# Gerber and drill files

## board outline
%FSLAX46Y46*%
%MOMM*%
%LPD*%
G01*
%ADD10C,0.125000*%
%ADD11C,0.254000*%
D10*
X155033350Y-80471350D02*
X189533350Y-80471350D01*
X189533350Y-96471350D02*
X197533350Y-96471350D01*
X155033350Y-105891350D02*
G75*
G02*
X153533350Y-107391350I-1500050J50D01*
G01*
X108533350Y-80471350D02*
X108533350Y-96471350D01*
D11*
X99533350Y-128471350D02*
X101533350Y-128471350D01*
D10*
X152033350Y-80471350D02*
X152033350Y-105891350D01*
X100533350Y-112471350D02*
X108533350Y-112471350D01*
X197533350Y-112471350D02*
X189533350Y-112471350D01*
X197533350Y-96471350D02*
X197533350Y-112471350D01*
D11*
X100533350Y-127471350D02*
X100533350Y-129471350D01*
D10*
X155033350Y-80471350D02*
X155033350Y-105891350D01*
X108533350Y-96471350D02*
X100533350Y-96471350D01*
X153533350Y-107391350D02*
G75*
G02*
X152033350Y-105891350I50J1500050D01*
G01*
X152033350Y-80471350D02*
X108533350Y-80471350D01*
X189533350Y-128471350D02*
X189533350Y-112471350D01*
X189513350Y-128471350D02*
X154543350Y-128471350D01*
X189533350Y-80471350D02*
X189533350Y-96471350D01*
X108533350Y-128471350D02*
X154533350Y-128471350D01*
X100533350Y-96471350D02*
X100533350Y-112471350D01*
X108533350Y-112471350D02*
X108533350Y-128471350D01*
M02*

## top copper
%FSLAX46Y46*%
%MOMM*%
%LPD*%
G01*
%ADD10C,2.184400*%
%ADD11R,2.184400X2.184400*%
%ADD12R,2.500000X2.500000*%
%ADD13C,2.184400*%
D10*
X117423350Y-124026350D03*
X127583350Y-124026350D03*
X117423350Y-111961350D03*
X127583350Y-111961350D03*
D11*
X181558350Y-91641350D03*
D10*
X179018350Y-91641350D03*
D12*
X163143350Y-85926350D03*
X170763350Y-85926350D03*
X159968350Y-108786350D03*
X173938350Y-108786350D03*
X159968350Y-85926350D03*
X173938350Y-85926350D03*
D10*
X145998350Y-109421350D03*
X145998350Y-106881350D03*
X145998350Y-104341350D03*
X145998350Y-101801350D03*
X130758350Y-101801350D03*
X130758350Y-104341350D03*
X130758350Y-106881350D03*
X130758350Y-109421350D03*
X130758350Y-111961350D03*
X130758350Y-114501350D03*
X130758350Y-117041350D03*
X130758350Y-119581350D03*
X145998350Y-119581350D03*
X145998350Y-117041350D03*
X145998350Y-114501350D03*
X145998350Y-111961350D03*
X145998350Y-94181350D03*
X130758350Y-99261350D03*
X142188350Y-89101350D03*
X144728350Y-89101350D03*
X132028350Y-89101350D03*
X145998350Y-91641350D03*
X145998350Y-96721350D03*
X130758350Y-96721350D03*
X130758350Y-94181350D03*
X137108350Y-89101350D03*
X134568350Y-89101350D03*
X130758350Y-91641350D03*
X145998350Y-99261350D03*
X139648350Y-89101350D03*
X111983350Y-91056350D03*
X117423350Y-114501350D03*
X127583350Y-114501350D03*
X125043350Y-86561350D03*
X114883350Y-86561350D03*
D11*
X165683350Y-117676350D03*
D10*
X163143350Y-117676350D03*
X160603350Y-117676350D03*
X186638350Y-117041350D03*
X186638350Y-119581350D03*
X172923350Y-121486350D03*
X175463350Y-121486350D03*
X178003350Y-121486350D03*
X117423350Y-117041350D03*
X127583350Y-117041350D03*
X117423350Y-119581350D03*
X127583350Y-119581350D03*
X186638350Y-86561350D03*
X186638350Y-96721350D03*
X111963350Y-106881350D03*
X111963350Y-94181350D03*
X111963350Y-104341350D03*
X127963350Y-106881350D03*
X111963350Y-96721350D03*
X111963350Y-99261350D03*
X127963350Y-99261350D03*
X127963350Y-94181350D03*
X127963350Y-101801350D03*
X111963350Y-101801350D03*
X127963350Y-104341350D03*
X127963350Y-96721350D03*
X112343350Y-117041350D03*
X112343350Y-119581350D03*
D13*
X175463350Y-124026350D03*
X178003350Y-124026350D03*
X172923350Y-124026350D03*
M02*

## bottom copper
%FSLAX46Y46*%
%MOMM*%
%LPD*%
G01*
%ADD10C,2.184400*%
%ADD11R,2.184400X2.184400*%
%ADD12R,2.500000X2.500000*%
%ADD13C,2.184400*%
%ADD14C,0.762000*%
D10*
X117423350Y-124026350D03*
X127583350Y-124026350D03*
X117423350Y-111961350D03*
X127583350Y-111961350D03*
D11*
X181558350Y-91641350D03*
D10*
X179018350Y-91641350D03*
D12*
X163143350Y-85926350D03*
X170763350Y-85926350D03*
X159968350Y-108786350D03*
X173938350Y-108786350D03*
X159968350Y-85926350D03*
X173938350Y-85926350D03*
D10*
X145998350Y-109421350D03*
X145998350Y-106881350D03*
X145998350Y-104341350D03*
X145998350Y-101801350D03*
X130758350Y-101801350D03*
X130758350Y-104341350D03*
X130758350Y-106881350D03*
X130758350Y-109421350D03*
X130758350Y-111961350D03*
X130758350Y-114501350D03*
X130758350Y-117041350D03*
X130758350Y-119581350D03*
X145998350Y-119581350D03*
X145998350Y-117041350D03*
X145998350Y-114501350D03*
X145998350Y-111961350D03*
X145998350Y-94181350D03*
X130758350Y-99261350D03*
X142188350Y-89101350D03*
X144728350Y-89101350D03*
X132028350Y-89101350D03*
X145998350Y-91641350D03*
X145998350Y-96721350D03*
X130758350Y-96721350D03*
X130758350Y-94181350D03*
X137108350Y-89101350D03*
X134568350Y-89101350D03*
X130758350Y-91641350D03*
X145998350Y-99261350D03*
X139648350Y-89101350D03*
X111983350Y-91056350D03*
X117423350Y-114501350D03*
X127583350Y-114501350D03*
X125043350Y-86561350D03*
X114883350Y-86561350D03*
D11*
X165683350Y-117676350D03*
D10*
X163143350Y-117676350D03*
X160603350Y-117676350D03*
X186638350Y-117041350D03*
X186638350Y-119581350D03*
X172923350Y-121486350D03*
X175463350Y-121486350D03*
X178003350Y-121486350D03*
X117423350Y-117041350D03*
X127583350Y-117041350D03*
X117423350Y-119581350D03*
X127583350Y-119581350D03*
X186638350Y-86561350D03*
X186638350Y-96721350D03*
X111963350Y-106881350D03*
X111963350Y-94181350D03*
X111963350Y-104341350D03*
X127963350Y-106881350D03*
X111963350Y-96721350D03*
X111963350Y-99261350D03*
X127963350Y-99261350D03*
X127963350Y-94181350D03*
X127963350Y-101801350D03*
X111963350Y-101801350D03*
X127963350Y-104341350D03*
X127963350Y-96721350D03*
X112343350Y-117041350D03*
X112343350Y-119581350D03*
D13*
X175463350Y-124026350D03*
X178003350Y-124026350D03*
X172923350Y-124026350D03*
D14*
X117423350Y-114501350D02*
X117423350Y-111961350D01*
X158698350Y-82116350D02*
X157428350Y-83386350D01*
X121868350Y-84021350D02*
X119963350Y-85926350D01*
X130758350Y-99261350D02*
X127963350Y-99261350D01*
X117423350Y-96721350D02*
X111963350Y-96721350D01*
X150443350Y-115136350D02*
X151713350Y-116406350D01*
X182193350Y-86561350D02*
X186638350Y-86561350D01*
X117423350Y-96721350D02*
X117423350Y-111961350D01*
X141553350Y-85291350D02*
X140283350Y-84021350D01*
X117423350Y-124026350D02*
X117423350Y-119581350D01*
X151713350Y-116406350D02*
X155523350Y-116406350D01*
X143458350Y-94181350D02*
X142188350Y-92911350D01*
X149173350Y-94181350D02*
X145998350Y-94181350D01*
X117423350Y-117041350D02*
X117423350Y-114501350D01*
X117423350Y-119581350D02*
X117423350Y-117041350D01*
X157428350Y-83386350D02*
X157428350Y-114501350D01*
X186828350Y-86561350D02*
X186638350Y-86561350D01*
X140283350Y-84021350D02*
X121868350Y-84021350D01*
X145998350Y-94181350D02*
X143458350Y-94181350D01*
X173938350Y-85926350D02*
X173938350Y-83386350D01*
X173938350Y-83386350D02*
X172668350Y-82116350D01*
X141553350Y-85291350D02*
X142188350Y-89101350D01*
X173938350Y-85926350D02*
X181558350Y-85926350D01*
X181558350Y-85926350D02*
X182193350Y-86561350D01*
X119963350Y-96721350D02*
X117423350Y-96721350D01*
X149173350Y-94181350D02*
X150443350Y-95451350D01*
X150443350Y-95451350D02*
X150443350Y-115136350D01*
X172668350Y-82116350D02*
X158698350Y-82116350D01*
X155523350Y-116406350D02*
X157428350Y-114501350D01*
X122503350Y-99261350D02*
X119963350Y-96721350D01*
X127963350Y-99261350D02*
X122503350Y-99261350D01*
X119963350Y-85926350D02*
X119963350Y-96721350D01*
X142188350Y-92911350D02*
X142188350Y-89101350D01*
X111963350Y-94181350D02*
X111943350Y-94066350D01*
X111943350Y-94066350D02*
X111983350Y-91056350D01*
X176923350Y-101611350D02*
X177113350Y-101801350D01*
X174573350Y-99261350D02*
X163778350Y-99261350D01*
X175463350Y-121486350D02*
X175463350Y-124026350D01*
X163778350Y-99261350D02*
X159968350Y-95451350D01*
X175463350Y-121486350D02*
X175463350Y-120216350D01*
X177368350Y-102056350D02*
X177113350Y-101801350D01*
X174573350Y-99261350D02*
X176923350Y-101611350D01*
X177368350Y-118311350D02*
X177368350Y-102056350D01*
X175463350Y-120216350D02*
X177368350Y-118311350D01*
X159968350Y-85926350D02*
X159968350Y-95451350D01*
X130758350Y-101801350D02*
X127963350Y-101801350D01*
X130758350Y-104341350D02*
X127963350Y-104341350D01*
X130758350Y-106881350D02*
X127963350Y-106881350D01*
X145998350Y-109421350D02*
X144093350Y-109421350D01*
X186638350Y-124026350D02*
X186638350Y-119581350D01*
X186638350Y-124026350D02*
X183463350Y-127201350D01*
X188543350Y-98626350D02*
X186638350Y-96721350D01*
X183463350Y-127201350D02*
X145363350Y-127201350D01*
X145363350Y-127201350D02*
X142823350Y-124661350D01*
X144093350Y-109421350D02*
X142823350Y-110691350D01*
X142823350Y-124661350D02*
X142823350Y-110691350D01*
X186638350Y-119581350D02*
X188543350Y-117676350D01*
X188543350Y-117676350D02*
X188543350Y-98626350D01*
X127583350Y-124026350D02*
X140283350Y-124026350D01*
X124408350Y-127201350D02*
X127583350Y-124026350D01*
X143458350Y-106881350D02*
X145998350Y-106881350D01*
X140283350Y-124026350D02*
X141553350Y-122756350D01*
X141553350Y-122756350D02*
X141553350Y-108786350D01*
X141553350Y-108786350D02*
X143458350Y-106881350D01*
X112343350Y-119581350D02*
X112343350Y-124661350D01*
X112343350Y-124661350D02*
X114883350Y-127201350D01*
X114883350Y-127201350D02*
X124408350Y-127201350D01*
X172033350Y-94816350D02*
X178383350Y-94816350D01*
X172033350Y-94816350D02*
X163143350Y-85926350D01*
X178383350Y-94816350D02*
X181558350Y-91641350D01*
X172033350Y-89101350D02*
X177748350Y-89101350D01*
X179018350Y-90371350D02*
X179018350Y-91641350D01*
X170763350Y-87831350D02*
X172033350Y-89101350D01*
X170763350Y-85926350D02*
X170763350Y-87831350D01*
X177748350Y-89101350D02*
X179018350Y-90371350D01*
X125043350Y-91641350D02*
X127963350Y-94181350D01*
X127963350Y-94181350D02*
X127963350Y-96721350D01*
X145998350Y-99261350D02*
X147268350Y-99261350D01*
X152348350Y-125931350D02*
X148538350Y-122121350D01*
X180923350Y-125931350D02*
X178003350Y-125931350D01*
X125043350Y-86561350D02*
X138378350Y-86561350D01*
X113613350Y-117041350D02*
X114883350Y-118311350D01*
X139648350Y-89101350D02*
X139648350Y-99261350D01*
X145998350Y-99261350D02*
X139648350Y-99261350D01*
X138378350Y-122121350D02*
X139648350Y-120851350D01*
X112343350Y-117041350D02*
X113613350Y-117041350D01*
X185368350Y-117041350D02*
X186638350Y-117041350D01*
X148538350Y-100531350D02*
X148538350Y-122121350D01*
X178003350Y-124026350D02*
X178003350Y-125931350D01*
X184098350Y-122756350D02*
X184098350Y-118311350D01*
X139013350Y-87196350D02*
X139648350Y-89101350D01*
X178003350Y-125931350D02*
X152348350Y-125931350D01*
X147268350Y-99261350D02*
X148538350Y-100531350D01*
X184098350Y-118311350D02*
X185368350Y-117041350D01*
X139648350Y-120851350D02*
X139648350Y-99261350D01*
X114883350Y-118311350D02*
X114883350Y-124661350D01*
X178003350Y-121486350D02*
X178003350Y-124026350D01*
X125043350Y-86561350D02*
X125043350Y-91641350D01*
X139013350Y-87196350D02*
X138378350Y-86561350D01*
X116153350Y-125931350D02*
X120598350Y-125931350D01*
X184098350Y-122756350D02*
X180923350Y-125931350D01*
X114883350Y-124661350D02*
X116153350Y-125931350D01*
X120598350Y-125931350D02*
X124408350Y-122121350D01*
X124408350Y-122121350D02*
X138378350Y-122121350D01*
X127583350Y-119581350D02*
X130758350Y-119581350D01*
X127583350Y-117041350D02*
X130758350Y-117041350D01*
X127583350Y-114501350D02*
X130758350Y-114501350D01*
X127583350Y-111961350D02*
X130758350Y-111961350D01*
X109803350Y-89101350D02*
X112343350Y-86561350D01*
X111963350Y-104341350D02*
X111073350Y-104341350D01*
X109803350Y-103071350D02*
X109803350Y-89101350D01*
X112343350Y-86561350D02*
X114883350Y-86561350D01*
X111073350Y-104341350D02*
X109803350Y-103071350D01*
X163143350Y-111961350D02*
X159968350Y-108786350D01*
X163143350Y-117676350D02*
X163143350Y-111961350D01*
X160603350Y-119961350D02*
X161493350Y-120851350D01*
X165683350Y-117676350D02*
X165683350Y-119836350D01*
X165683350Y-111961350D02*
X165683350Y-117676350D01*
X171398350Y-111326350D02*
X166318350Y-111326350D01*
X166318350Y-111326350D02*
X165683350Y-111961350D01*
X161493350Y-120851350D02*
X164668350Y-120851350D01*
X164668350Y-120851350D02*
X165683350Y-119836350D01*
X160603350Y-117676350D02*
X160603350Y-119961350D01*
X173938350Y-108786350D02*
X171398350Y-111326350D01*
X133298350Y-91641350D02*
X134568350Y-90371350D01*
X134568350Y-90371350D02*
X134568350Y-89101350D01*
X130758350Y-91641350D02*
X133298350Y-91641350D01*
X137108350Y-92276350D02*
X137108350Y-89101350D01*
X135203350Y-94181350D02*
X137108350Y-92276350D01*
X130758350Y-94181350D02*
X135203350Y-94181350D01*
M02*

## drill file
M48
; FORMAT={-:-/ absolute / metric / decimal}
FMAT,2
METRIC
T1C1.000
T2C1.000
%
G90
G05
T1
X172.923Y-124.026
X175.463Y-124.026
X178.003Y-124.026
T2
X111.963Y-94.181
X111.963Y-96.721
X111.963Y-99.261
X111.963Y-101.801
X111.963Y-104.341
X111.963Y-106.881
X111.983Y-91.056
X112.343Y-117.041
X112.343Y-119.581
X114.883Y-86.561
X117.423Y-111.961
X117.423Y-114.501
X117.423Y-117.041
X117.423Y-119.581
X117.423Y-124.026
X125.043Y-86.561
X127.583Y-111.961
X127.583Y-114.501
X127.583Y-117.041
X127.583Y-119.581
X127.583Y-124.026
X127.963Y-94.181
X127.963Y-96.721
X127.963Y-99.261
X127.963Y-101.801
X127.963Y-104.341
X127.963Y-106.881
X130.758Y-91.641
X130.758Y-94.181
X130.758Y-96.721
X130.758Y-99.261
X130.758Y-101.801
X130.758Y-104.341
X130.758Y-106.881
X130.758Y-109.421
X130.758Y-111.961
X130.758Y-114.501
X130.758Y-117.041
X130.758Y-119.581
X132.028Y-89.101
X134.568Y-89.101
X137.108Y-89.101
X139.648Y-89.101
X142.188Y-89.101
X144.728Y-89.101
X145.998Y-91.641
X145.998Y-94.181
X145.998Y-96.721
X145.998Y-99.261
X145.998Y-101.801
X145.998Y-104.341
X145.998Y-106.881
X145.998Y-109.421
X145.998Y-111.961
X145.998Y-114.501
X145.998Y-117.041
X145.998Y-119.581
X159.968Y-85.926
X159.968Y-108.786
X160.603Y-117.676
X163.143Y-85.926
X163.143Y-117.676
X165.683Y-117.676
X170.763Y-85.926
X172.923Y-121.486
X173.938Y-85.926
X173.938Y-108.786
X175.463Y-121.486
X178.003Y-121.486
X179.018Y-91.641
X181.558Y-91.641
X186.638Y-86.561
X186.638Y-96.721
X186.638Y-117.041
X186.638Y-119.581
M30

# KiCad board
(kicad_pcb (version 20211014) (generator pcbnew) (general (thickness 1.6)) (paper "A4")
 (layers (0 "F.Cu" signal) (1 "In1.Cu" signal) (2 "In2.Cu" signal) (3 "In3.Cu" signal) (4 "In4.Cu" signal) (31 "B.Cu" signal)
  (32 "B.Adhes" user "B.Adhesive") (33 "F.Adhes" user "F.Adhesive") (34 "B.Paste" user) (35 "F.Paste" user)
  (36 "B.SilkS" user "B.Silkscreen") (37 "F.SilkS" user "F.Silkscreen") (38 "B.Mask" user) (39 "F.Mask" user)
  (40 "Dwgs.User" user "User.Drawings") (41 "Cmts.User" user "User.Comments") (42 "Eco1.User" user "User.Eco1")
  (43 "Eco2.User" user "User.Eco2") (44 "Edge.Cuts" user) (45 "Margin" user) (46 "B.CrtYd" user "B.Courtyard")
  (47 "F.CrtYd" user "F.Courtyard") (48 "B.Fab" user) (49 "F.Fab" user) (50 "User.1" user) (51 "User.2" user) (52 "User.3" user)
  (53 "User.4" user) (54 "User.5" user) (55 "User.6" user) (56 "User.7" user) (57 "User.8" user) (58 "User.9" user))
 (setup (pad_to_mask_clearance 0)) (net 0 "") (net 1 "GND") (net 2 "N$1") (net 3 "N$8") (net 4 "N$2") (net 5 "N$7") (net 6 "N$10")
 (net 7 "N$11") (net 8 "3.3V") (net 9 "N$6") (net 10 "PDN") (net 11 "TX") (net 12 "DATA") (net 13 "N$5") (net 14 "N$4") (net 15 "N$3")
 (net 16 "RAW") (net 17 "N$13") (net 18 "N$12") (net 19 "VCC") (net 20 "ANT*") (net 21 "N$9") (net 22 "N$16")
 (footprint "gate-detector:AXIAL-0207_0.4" (layer "F.Cu") (at 122.50335 124.02635)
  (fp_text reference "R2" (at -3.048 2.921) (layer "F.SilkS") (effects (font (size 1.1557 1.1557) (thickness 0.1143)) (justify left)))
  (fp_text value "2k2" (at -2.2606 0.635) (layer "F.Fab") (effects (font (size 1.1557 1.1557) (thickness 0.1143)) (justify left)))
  (pad "1" thru_hole circle (at -5.08 0) (size 2.1844 2.1844) (drill 1) (layers *.Cu *.Mask) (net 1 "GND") (solder_mask_margin 0.0508))
  (pad "2" thru_hole circle (at 5.08 0) (size 2.1844 2.1844) (drill 1) (layers *.Cu *.Mask) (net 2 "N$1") (solder_mask_margin 0.0508)))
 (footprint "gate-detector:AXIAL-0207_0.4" (layer "F.Cu") (at 122.50335 111.96135)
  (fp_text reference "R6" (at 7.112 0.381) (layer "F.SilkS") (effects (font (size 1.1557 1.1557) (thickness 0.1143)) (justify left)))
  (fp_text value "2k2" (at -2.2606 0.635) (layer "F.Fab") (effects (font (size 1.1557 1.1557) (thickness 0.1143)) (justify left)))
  (pad "1" thru_hole circle (at -5.08 0) (size 2.1844 2.1844) (drill 1) (layers *.Cu *.Mask) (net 1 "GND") (solder_mask_margin 0.0508))
  (pad "2" thru_hole circle (at 5.08 0) (size 2.1844 2.1844) (drill 1) (layers *.Cu *.Mask) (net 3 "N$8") (solder_mask_margin 0.0508)))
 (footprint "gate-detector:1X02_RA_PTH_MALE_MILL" (layer "F.Cu") (at 181.55835 91.64135 180)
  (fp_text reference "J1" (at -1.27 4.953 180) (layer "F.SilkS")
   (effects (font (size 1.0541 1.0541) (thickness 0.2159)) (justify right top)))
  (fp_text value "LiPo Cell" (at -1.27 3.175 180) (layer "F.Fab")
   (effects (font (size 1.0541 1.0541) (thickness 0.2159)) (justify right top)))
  (pad "1" thru_hole rect (at 0 0 270) (size 2.1844 2.1844) (drill 1) (layers *.Cu *.Mask) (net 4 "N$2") (solder_mask_margin 0.0508))
  (pad "2" thru_hole circle (at 2.54 0 270) (size 2.1844 2.1844) (drill 1) (layers *.Cu *.Mask) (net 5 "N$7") (solder_mask_margin 0.0508)))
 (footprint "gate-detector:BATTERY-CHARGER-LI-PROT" (layer "F.Cu") (at 166.95335 96.72135 90)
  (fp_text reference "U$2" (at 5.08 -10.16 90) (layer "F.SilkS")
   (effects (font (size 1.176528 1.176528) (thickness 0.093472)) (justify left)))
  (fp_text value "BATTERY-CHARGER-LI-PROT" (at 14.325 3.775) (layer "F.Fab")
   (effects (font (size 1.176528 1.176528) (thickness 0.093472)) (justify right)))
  (pad "B+" thru_hole rect (at 10.795 -3.81 90) (size 2.5 2.5) (drill 1) (layers *.Cu *.Mask) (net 4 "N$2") (solder_mask_margin 0.0508))
  (pad "B-" thru_hole rect (at 10.795 3.81 90) (size 2.5 2.5) (drill 1) (layers *.Cu *.Mask) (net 5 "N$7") (solder_mask_margin 0.0508))
  (pad "IN+" thru_hole rect (at -12.065 -6.985 90) (size 2.5 2.5) (drill 1) (layers *.Cu *.Mask) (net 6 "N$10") (solder_mask_margin 0.0508))
  (pad "IN-" thru_hole rect (at -12.065 6.985 90) (size 2.5 2.5) (drill 1) (layers *.Cu *.Mask) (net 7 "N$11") (solder_mask_margin 0.0508))
  (pad "OUT+" thru_hole rect (at 10.795 -6.985 90) (size 2.5 2.5) (drill 1) (layers *.Cu *.Mask) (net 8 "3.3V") (solder_mask_margin 0.0508))
  (pad "OUT-" thru_hole rect (at 10.795 6.985 90) (size 2.5 2.5) (drill 1) (layers *.Cu *.Mask) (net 1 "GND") (solder_mask_margin 0.0508)))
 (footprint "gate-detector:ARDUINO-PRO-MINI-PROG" (layer "F.Cu") (at 138.37835 100.53135 -90)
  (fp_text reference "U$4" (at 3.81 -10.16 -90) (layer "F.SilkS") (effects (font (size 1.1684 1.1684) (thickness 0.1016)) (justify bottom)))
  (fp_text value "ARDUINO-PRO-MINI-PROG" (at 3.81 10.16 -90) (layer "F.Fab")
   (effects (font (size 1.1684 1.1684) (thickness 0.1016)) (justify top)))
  (pad "A0" thru_hole circle (at 8.89 -7.62 270) (size 2.1844 2.1844) (drill 1) (layers *.Cu *.Mask) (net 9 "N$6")
   (solder_mask_margin 0.0508))
  (pad "A1" thru_hole circle (at 6.35 -7.62 270) (size 2.1844 2.1844) (drill 1) (layers *.Cu *.Mask) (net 2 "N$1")
   (solder_mask_margin 0.0508))
  (pad "A2" thru_hole circle (at 3.81 -7.62 270) (size 2.1844 2.1844) (drill 1) (layers *.Cu *.Mask) (solder_mask_margin 0.0508))
  (pad "A3" thru_hole circle (at 1.27 -7.62 270) (size 2.1844 2.1844) (drill 1) (layers *.Cu *.Mask) (solder_mask_margin 0.0508))
  (pad "D2" thru_hole circle (at 1.27 7.62 270) (size 2.1844 2.1844) (drill 1) (layers *.Cu *.Mask) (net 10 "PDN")
   (solder_mask_margin 0.0508))
  (pad "D3" thru_hole circle (at 3.81 7.62 270) (size 2.1844 2.1844) (drill 1) (layers *.Cu *.Mask) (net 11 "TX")
   (solder_mask_margin 0.0508))
  (pad "D4" thru_hole circle (at 6.35 7.62 270) (size 2.1844 2.1844) (drill 1) (layers *.Cu *.Mask) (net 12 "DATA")
   (solder_mask_margin 0.0508))
  (pad "D5" thru_hole circle (at 8.89 7.62 270) (size 2.1844 2.1844) (drill 1) (layers *.Cu *.Mask) (solder_mask_margin 0.0508))
  (pad "D6" thru_hole circle (at 11.43 7.62 270) (size 2.1844 2.1844) (drill 1) (layers *.Cu *.Mask) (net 3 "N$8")
   (solder_mask_margin 0.0508))
  (pad "D7" thru_hole circle (at 13.97 7.62 270) (size 2.1844 2.1844) (drill 1) (layers *.Cu *.Mask) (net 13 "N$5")
   (solder_mask_margin 0.0508))
  (pad "D8" thru_hole circle (at 16.51 7.62 270) (size 2.1844 2.1844) (drill 1) (layers *.Cu *.Mask) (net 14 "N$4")
   (solder_mask_margin 0.0508))
  (pad "D9" thru_hole circle (at 19.05 7.62 270) (size 2.1844 2.1844) (drill 1) (layers *.Cu *.Mask) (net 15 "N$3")
   (solder_mask_margin 0.0508))
  (pad "D10" thru_hole circle (at 19.05 -7.62 270) (size 2.1844 2.1844) (drill 1) (layers *.Cu *.Mask) (solder_mask_margin 0.0508))
  (pad "D11" thru_hole circle (at 16.51 -7.62 270) (size 2.1844 2.1844) (drill 1) (layers *.Cu *.Mask) (solder_mask_margin 0.0508))
  (pad "D12" thru_hole circle (at 13.97 -7.62 270) (size 2.1844 2.1844) (drill 1) (layers *.Cu *.Mask) (solder_mask_margin 0.0508))
  (pad "D13" thru_hole circle (at 11.43 -7.62 270) (size 2.1844 2.1844) (drill 1) (layers *.Cu *.Mask) (solder_mask_margin 0.0508))
  (pad "GND@1" thru_hole circle (at -6.35 -7.62 270) (size 2.1844 2.1844) (drill 1) (layers *.Cu *.Mask) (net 1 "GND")
   (solder_mask_margin 0.0508))
  (pad "GND@2" thru_hole circle (at -1.27 7.62 270) (size 2.1844 2.1844) (drill 1) (layers *.Cu *.Mask) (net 1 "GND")
   (solder_mask_margin 0.0508))
  (pad "GND@3" thru_hole circle (at -11.43 -3.81 270) (size 2.1844 2.1844) (drill 1) (layers *.Cu *.Mask) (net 1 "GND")
   (solder_mask_margin 0.0508))
  (pad "P_CTS" thru_hole circle (at -11.43 -6.35 270) (size 2.1844 2.1844) (drill 1) (layers *.Cu *.Mask) (solder_mask_margin 0.0508))
  (pad "P_DTR" thru_hole circle (at -11.43 6.35 270) (size 2.1844 2.1844) (drill 1) (layers *.Cu *.Mask) (solder_mask_margin 0.0508))
  (pad "RAW" thru_hole circle (at -8.89 -7.62 270) (size 2.1844 2.1844) (drill 1) (layers *.Cu *.Mask) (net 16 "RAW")
   (solder_mask_margin 0.0508))
  (pad "RST@1" thru_hole circle (at -3.81 -7.62 270) (size 2.1844 2.1844) (drill 1) (layers *.Cu *.Mask) (solder_mask_margin 0.0508))
  (pad "RST@2" thru_hole circle (at -3.81 7.62 270) (size 2.1844 2.1844) (drill 1) (layers *.Cu *.Mask) (solder_mask_margin 0.0508))
  (pad "RX0@1" thru_hole circle (at -6.35 7.62 270) (size 2.1844 2.1844) (drill 1) (layers *.Cu *.Mask) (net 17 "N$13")
   (solder_mask_margin 0.0508))
  (pad "RX1@2" thru_hole circle (at -11.43 1.27 270) (size 2.1844 2.1844) (drill 1) (layers *.Cu *.Mask) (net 17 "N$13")
   (solder_mask_margin 0.0508))
  (pad "TX0@2" thru_hole circle (at -11.43 3.81 270) (size 2.1844 2.1844) (drill 1) (layers *.Cu *.Mask) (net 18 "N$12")
   (solder_mask_margin 0.0508))
  (pad "TX1@1" thru_hole circle (at -8.89 7.62 270) (size 2.1844 2.1844) (drill 1) (layers *.Cu *.Mask) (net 18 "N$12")
   (solder_mask_margin 0.0508))
  (pad "VCC@1" thru_hole circle (at -1.27 -7.62 270) (size 2.1844 2.1844) (drill 1) (layers *.Cu *.Mask) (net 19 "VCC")
   (solder_mask_margin 0.0508))
  (pad "VCC@2" thru_hole circle (at -11.43 -1.27 270) (size 2.1844 2.1844) (drill 1) (layers *.Cu *.Mask) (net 19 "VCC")
   (solder_mask_margin 0.0508)))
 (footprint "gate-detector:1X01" (layer "F.Cu") (at 111.98335 91.05635)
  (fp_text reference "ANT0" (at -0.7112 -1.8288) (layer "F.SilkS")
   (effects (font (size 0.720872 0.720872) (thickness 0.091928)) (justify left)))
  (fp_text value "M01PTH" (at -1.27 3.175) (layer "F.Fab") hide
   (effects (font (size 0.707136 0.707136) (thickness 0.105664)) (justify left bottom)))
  (pad "1" thru_hole circle (at 0 0 90) (size 2.1844 2.1844) (drill 1) (layers *.Cu *.Mask) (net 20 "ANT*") (solder_mask_margin 0.0508)))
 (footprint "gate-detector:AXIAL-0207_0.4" (layer "F.Cu") (at 122.50335 114.50135)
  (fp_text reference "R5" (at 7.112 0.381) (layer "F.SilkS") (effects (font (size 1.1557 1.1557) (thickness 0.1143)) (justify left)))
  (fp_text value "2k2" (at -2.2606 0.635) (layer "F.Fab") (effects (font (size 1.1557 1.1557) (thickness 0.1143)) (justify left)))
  (pad "1" thru_hole circle (at -5.08 0) (size 2.1844 2.1844) (drill 1) (layers *.Cu *.Mask) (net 1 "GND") (solder_mask_margin 0.0508))
  (pad "2" thru_hole circle (at 5.08 0) (size 2.1844 2.1844) (drill 1) (layers *.Cu *.Mask) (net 13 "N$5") (solder_mask_margin 0.0508)))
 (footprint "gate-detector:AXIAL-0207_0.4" (layer "F.Cu") (at 119.96335 86.56135 180)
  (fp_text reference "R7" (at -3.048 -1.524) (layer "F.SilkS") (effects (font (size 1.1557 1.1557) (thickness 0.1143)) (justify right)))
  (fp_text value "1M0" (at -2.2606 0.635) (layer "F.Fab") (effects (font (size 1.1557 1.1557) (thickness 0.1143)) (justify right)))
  (pad "1" thru_hole circle (at -5.08 0 180) (size 2.1844 2.1844) (drill 1) (layers *.Cu *.Mask) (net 19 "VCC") (solder_mask_margin 0.0508))
  (pad "2" thru_hole circle (at 5.08 0 180) (size 2.1844 2.1844) (drill 1) (layers *.Cu *.Mask) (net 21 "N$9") (solder_mask_margin 0.0508)))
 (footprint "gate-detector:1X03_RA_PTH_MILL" (layer "F.Cu") (at 165.68335 117.67635 180)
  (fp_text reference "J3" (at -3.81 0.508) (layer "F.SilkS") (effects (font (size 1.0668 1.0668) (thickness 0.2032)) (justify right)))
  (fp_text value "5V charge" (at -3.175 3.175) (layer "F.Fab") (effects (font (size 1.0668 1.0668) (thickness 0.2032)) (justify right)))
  (pad "1" thru_hole rect (at 0 0 270) (size 2.1844 2.1844) (drill 1) (layers *.Cu *.Mask) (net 7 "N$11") (solder_mask_margin 0.0508))
  (pad "2" thru_hole circle (at 2.54 0 270) (size 2.1844 2.1844) (drill 1) (layers *.Cu *.Mask) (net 6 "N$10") (solder_mask_margin 0.0508))
  (pad "3" thru_hole circle (at 5.08 0 270) (size 2.1844 2.1844) (drill 1) (layers *.Cu *.Mask) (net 7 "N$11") (solder_mask_margin 0.0508)))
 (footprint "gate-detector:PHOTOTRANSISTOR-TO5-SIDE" (layer "F.Cu") (at 186.63835 118.31135)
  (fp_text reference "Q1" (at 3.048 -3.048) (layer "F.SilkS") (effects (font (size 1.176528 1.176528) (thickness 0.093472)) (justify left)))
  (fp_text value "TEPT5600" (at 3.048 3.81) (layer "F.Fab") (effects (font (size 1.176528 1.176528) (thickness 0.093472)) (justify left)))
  (pad "C" thru_hole circle (at 0 -1.27) (size 2.1844 2.1844) (drill 1) (layers *.Cu *.Mask) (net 19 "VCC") (solder_mask_margin 0.0508))
  (pad "E" thru_hole circle (at 0 1.27) (size 2.1844 2.1844) (drill 1) (layers *.Cu *.Mask) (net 9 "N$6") (solder_mask_margin 0.0508)))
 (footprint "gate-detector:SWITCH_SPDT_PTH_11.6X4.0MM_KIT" (layer "F.Cu") (at 175.46335 121.48635 90)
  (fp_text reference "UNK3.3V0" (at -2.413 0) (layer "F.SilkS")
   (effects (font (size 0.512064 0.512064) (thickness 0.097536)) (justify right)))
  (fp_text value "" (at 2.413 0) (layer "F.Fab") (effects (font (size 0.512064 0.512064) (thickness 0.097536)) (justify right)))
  (pad "1" thru_hole circle (at 0 -2.54 90) (size 2.1844 2.1844) (drill 1) (layers *.Cu) (solder_mask_margin 0.0508))
  (pad "2" thru_hole circle (at 0 0 90) (size 2.1844 2.1844) (drill 1) (layers *.Cu) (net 8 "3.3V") (solder_mask_margin 0.0508))
  (pad "3" thru_hole circle (at 0 2.54 90) (size 2.1844 2.1844) (drill 1) (layers *.Cu) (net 19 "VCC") (solder_mask_margin 0.0508)))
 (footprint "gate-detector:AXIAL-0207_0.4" (layer "F.Cu") (at 122.50335 117.04135)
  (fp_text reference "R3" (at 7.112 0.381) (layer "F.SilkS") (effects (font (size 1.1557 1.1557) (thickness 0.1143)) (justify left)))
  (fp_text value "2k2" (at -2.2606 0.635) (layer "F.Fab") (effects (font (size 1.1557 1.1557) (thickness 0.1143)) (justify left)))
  (pad "1" thru_hole circle (at -5.08 0) (size 2.1844 2.1844) (drill 1) (layers *.Cu *.Mask) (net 1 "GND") (solder_mask_margin 0.0508))
  (pad "2" thru_hole circle (at 5.08 0) (size 2.1844 2.1844) (drill 1) (layers *.Cu *.Mask) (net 14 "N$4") (solder_mask_margin 0.0508)))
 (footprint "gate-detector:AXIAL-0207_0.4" (layer "F.Cu") (at 122.50335 119.58135)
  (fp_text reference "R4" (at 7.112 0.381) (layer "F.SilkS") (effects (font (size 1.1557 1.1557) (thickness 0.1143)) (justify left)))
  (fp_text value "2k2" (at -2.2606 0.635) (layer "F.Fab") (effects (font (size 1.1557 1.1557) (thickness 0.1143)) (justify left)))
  (pad "1" thru_hole circle (at -5.08 0) (size 2.1844 2.1844) (drill 1) (layers *.Cu *.Mask) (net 1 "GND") (solder_mask_margin 0.0508))
  (pad "2" thru_hole circle (at 5.08 0) (size 2.1844 2.1844) (drill 1) (layers *.Cu *.Mask) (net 15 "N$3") (solder_mask_margin 0.0508)))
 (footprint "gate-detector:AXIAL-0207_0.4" (layer "F.Cu") (at 186.63835 91.64135 -90)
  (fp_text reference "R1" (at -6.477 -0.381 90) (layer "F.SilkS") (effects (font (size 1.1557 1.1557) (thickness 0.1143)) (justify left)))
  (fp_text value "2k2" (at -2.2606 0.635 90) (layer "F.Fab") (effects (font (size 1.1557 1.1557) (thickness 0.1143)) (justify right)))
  (pad "1" thru_hole circle (at -5.08 0 270) (size 2.1844 2.1844) (drill 1) (layers *.Cu *.Mask) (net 1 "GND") (solder_mask_margin 0.0508))
  (pad "2" thru_hole circle (at 5.08 0 270) (size 2.1844 2.1844) (drill 1) (layers *.Cu *.Mask) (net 9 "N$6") (solder_mask_margin 0.0508)))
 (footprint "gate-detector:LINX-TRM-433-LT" (layer "F.Cu") (at 119.96335 101.80135)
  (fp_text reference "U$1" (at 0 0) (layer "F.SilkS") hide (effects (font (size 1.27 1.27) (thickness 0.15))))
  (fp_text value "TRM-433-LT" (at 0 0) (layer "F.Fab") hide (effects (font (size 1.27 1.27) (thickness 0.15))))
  (pad "ANALOG" thru_hole circle (at -8 5.08) (size 2.1844 2.1844) (drill 1) (layers *.Cu *.Mask) (solder_mask_margin 0.0508))
  (pad "ANT" thru_hole circle (at -8 -7.62) (size 2.1844 2.1844) (drill 1) (layers *.Cu *.Mask) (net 20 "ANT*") (solder_mask_margin 0.0508))
  (pad "AREF" thru_hole circle (at -8 2.54) (size 2.1844 2.1844) (drill 1) (layers *.Cu *.Mask) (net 21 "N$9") (solder_mask_margin 0.0508))
  (pad "DATA" thru_hole circle (at 8 5.08) (size 2.1844 2.1844) (drill 1) (layers *.Cu *.Mask) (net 12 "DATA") (solder_mask_margin 0.0508))
  (pad "GND" thru_hole circle (at -8 -5.08) (size 2.1844 2.1844) (drill 1) (layers *.Cu *.Mask) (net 1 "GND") (solder_mask_margin 0.0508))
  (pad "GND@1" thru_hole circle (at -8 -2.54) (size 2.1844 2.1844) (drill 1) (layers *.Cu *.Mask) (solder_mask_margin 0.0508))
  (pad "GND@2" thru_hole circle (at 8 -2.54) (size 2.1844 2.1844) (drill 1) (layers *.Cu *.Mask) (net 1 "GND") (solder_mask_margin 0.0508))
  (pad "LADJ" thru_hole circle (at 8 -7.62) (size 2.1844 2.1844) (drill 1) (layers *.Cu *.Mask) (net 19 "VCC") (solder_mask_margin 0.0508))
  (pad "PDN" thru_hole circle (at 8 0) (size 2.1844 2.1844) (drill 1) (layers *.Cu *.Mask) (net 10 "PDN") (solder_mask_margin 0.0508))
  (pad "RSSI" thru_hole circle (at -8 0) (size 2.1844 2.1844) (drill 1) (layers *.Cu *.Mask) (solder_mask_margin 0.0508))
  (pad "T/~R" thru_hole circle (at 8 2.54) (size 2.1844 2.1844) (drill 1) (layers *.Cu *.Mask) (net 11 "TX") (solder_mask_margin 0.0508))
  (pad "VCC" thru_hole circle (at 8 -5.08) (size 2.1844 2.1844) (drill 1) (layers *.Cu *.Mask) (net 19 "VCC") (solder_mask_margin 0.0508)))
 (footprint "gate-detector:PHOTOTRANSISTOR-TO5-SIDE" (layer "B.Cu") (at 112.34335 118.31135 180)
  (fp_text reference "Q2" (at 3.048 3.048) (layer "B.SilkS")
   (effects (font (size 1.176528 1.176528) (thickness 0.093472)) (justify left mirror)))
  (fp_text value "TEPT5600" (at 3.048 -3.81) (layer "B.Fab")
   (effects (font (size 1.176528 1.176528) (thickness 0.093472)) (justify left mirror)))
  (pad "C" thru_hole circle (at 0 1.27 180) (size 2.1844 2.1844) (drill 1) (layers *.Cu *.Mask) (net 19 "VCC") (solder_mask_margin 0.0508))
  (pad "E" thru_hole circle (at 0 -1.27 180) (size 2.1844 2.1844) (drill 1) (layers *.Cu *.Mask) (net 2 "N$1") (solder_mask_margin 0.0508)))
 (gr_line (start 155.03335 80.47135) (end 189.53335 80.47135) (layer "Edge.Cuts") (width 0.125))
 (gr_line (start 189.53335 96.47135) (end 197.53335 96.47135) (layer "Edge.Cuts") (width 0.125))
 (gr_arc (start 155.03335 105.89135) (mid 154.59401 106.95201) (end 153.53335 107.39135) (layer "Edge.Cuts") (width 0.125))
 (gr_line (start 108.53335 80.47135) (end 108.53335 96.47135) (layer "Edge.Cuts") (width 0.125))
 (gr_line (start 99.53335 128.47135) (end 101.53335 128.47135) (layer "Edge.Cuts") (width 0.254))
 (gr_line (start 152.03335 80.47135) (end 152.03335 105.89135) (layer "Edge.Cuts") (width 0.125))
 (gr_line (start 100.53335 112.47135) (end 108.53335 112.47135) (layer "Edge.Cuts") (width 0.125))
 (gr_line (start 197.53335 112.47135) (end 189.53335 112.47135) (layer "Edge.Cuts") (width 0.125))
 (gr_line (start 197.53335 96.47135) (end 197.53335 112.47135) (layer "Edge.Cuts") (width 0.125))
 (gr_line (start 100.53335 127.47135) (end 100.53335 129.47135) (layer "Edge.Cuts") (width 0.254))
 (gr_line (start 155.03335 80.47135) (end 155.03335 105.89135) (layer "Edge.Cuts") (width 0.125))
 (gr_line (start 108.53335 96.47135) (end 100.53335 96.47135) (layer "Edge.Cuts") (width 0.125))
 (gr_arc (start 153.53335 107.39135) (mid 152.47269 106.95201) (end 152.03335 105.89135) (layer "Edge.Cuts") (width 0.125))
 (gr_line (start 152.03335 80.47135) (end 108.53335 80.47135) (layer "Edge.Cuts") (width 0.125))
 (gr_line (start 189.53335 128.47135) (end 189.53335 112.47135) (layer "Edge.Cuts") (width 0.125))
 (gr_line (start 189.51335 128.47135) (end 154.54335 128.47135) (layer "Edge.Cuts") (width 0.125))
 (gr_line (start 189.53335 80.47135) (end 189.53335 96.47135) (layer "Edge.Cuts") (width 0.125))
 (gr_line (start 108.53335 128.47135) (end 154.53335 128.47135) (layer "Edge.Cuts") (width 0.125))
 (gr_line (start 100.53335 96.47135) (end 100.53335 112.47135) (layer "Edge.Cuts") (width 0.125))
 (gr_line (start 108.53335 112.47135) (end 108.53335 128.47135) (layer "Edge.Cuts") (width 0.125))
 (segment (start 117.42335 114.50135) (end 117.42335 111.96135) (width 0.762) (layer "B.Cu") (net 1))
 (segment (start 158.69835 82.11635) (end 157.42835 83.38635) (width 0.762) (layer "B.Cu") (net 1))
 (segment (start 121.86835 84.02135) (end 119.96335 85.92635) (width 0.762) (layer "B.Cu") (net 1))
 (segment (start 130.75835 99.26135) (end 127.96335 99.26135) (width 0.762) (layer "B.Cu") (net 1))
 (segment (start 117.42335 96.72135) (end 111.96335 96.72135) (width 0.762) (layer "B.Cu") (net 1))
 (segment (start 150.44335 115.13635) (end 151.71335 116.40635) (width 0.762) (layer "B.Cu") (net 1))
 (segment (start 182.19335 86.56135) (end 186.63835 86.56135) (width 0.762) (layer "B.Cu") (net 1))
 (segment (start 117.42335 96.72135) (end 117.42335 111.96135) (width 0.762) (layer "B.Cu") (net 1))
 (segment (start 141.55335 85.29135) (end 140.28335 84.02135) (width 0.762) (layer "B.Cu") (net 1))
 (segment (start 117.42335 124.02635) (end 117.42335 119.58135) (width 0.762) (layer "B.Cu") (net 1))
 (segment (start 151.71335 116.40635) (end 155.52335 116.40635) (width 0.762) (layer "B.Cu") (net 1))
 (segment (start 143.45835 94.18135) (end 142.18835 92.91135) (width 0.762) (layer "B.Cu") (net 1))
 (segment (start 149.17335 94.18135) (end 145.99835 94.18135) (width 0.762) (layer "B.Cu") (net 1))
 (segment (start 117.42335 117.04135) (end 117.42335 114.50135) (width 0.762) (layer "B.Cu") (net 1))
 (segment (start 117.42335 119.58135) (end 117.42335 117.04135) (width 0.762) (layer "B.Cu") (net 1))
 (segment (start 157.42835 83.38635) (end 157.42835 114.50135) (width 0.762) (layer "B.Cu") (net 1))
 (segment (start 186.82835 86.56135) (end 186.63835 86.56135) (width 0.762) (layer "B.Cu") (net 1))
 (segment (start 140.28335 84.02135) (end 121.86835 84.02135) (width 0.762) (layer "B.Cu") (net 1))
 (segment (start 145.99835 94.18135) (end 143.45835 94.18135) (width 0.762) (layer "B.Cu") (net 1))
 (segment (start 173.93835 85.92635) (end 173.93835 83.38635) (width 0.762) (layer "B.Cu") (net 1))
 (segment (start 173.93835 83.38635) (end 172.66835 82.11635) (width 0.762) (layer "B.Cu") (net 1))
 (segment (start 141.55335 85.29135) (end 142.18835 89.10135) (width 0.762) (layer "B.Cu") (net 1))
 (segment (start 173.93835 85.92635) (end 181.55835 85.92635) (width 0.762) (layer "B.Cu") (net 1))
 (segment (start 181.55835 85.92635) (end 182.19335 86.56135) (width 0.762) (layer "B.Cu") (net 1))
 (segment (start 119.96335 96.72135) (end 117.42335 96.72135) (width 0.762) (layer "B.Cu") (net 1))
 (segment (start 149.17335 94.18135) (end 150.44335 95.45135) (width 0.762) (layer "B.Cu") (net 1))
 (segment (start 150.44335 95.45135) (end 150.44335 115.13635) (width 0.762) (layer "B.Cu") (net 1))
 (segment (start 172.66835 82.11635) (end 158.69835 82.11635) (width 0.762) (layer "B.Cu") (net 1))
 (segment (start 155.52335 116.40635) (end 157.42835 114.50135) (width 0.762) (layer "B.Cu") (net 1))
 (segment (start 122.50335 99.26135) (end 119.96335 96.72135) (width 0.762) (layer "B.Cu") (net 1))
 (segment (start 127.96335 99.26135) (end 122.50335 99.26135) (width 0.762) (layer "B.Cu") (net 1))
 (segment (start 119.96335 85.92635) (end 119.96335 96.72135) (width 0.762) (layer "B.Cu") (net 1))
 (segment (start 142.18835 92.91135) (end 142.18835 89.10135) (width 0.762) (layer "B.Cu") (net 1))
 (segment (start 111.96335 94.18135) (end 111.94335 94.06635) (width 0.762) (layer "B.Cu") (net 20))
 (segment (start 111.94335 94.06635) (end 111.98335 91.05635) (width 0.762) (layer "B.Cu") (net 20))
 (via (at 175.46335 124.02635) (size 2.1844) (drill 1) (layers "F.Cu" "B.Cu") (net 8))
 (segment (start 176.92335 101.61135) (end 177.11335 101.80135) (width 0.762) (layer "B.Cu") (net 8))
 (segment (start 174.57335 99.26135) (end 163.77835 99.26135) (width 0.762) (layer "B.Cu") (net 8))
 (segment (start 175.46335 121.48635) (end 175.46335 124.02635) (width 0.762) (layer "B.Cu") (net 8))
 (segment (start 163.77835 99.26135) (end 159.96835 95.45135) (width 0.762) (layer "B.Cu") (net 8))
 (segment (start 175.46335 121.48635) (end 175.46335 120.21635) (width 0.762) (layer "B.Cu") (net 8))
 (segment (start 177.36835 102.05635) (end 177.11335 101.80135) (width 0.762) (layer "B.Cu") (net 8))
 (segment (start 174.57335 99.26135) (end 176.92335 101.61135) (width 0.762) (layer "B.Cu") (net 8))
 (segment (start 177.36835 118.31135) (end 177.36835 102.05635) (width 0.762) (layer "B.Cu") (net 8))
 (segment (start 175.46335 120.21635) (end 177.36835 118.31135) (width 0.762) (layer "B.Cu") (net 8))
 (segment (start 159.96835 85.92635) (end 159.96835 95.45135) (width 0.762) (layer "B.Cu") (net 8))
 (segment (start 130.75835 101.80135) (end 127.96335 101.80135) (width 0.762) (layer "B.Cu") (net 10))
 (segment (start 130.75835 104.34135) (end 127.96335 104.34135) (width 0.762) (layer "B.Cu") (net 11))
 (segment (start 130.75835 106.88135) (end 127.96335 106.88135) (width 0.762) (layer "B.Cu") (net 12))
 (segment (start 145.99835 109.42135) (end 144.09335 109.42135) (width 0.762) (layer "B.Cu") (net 9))
 (segment (start 186.63835 124.02635) (end 186.63835 119.58135) (width 0.762) (layer "B.Cu") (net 9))
 (segment (start 186.63835 124.02635) (end 183.46335 127.20135) (width 0.762) (layer "B.Cu") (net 9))
 (segment (start 188.54335 98.62635) (end 186.63835 96.72135) (width 0.762) (layer "B.Cu") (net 9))
 (segment (start 183.46335 127.20135) (end 145.36335 127.20135) (width 0.762) (layer "B.Cu") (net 9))
 (segment (start 145.36335 127.20135) (end 142.82335 124.66135) (width 0.762) (layer "B.Cu") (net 9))
 (segment (start 144.09335 109.42135) (end 142.82335 110.69135) (width 0.762) (layer "B.Cu") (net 9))
 (segment (start 142.82335 124.66135) (end 142.82335 110.69135) (width 0.762) (layer "B.Cu") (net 9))
 (segment (start 186.63835 119.58135) (end 188.54335 117.67635) (width 0.762) (layer "B.Cu") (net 9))
 (segment (start 188.54335 117.67635) (end 188.54335 98.62635) (width 0.762) (layer "B.Cu") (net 9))
 (segment (start 127.58335 124.02635) (end 140.28335 124.02635) (width 0.762) (layer "B.Cu") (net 2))
 (segment (start 124.40835 127.20135) (end 127.58335 124.02635) (width 0.762) (layer "B.Cu") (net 2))
 (segment (start 143.45835 106.88135) (end 145.99835 106.88135) (width 0.762) (layer "B.Cu") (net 2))
 (segment (start 140.28335 124.02635) (end 141.55335 122.75635) (width 0.762) (layer "B.Cu") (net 2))
 (segment (start 141.55335 122.75635) (end 141.55335 108.78635) (width 0.762) (layer "B.Cu") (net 2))
 (segment (start 141.55335 108.78635) (end 143.45835 106.88135) (width 0.762) (layer "B.Cu") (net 2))
 (segment (start 112.34335 119.58135) (end 112.34335 124.66135) (width 0.762) (layer "B.Cu") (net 2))
 (segment (start 112.34335 124.66135) (end 114.88335 127.20135) (width 0.762) (layer "B.Cu") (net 2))
 (segment (start 114.88335 127.20135) (end 124.40835 127.20135) (width 0.762) (layer "B.Cu") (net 2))
 (segment (start 172.03335 94.81635) (end 178.38335 94.81635) (width 0.762) (layer "B.Cu") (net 4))
 (segment (start 172.03335 94.81635) (end 163.14335 85.92635) (width 0.762) (layer "B.Cu") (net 4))
 (segment (start 178.38335 94.81635) (end 181.55835 91.64135) (width 0.762) (layer "B.Cu") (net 4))
 (segment (start 172.03335 89.10135) (end 177.74835 89.10135) (width 0.762) (layer "B.Cu") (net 5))
 (segment (start 179.01835 90.37135) (end 179.01835 91.64135) (width 0.762) (layer "B.Cu") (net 5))
 (segment (start 170.76335 87.83135) (end 172.03335 89.10135) (width 0.762) (layer "B.Cu") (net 5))
 (segment (start 170.76335 85.92635) (end 170.76335 87.83135) (width 0.762) (layer "B.Cu") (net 5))
 (segment (start 177.74835 89.10135) (end 179.01835 90.37135) (width 0.762) (layer "B.Cu") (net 5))
 (via (at 178.00335 124.02635) (size 2.1844) (drill 1) (layers "F.Cu" "B.Cu") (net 19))
 (segment (start 125.04335 91.64135) (end 127.96335 94.18135) (width 0.762) (layer "B.Cu") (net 19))
 (segment (start 127.96335 94.18135) (end 127.96335 96.72135) (width 0.762) (layer "B.Cu") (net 19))
 (segment (start 145.99835 99.26135) (end 147.26835 99.26135) (width 0.762) (layer "B.Cu") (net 19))
 (segment (start 152.34835 125.93135) (end 148.53835 122.12135) (width 0.762) (layer "B.Cu") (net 19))
 (segment (start 180.92335 125.93135) (end 178.00335 125.93135) (width 0.762) (layer "B.Cu") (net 19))
 (segment (start 125.04335 86.56135) (end 138.37835 86.56135) (width 0.762) (layer "B.Cu") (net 19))
 (segment (start 113.61335 117.04135) (end 114.88335 118.31135) (width 0.762) (layer "B.Cu") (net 19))
 (segment (start 139.64835 89.10135) (end 139.64835 99.26135) (width 0.762) (layer "B.Cu") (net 19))
 (segment (start 145.99835 99.26135) (end 139.64835 99.26135) (width 0.762) (layer "B.Cu") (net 19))
 (segment (start 138.37835 122.12135) (end 139.64835 120.85135) (width 0.762) (layer "B.Cu") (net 19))
 (segment (start 112.34335 117.04135) (end 113.61335 117.04135) (width 0.762) (layer "B.Cu") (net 19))
 (segment (start 185.36835 117.04135) (end 186.63835 117.04135) (width 0.762) (layer "B.Cu") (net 19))
 (segment (start 148.53835 100.53135) (end 148.53835 122.12135) (width 0.762) (layer "B.Cu") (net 19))
 (segment (start 178.00335 124.02635) (end 178.00335 125.93135) (width 0.762) (layer "B.Cu") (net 19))
 (segment (start 184.09835 122.75635) (end 184.09835 118.31135) (width 0.762) (layer "B.Cu") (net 19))
 (segment (start 139.01335 87.19635) (end 139.64835 89.10135) (width 0.762) (layer "B.Cu") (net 19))
 (segment (start 178.00335 125.93135) (end 152.34835 125.93135) (width 0.762) (layer "B.Cu") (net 19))
 (segment (start 147.26835 99.26135) (end 148.53835 100.53135) (width 0.762) (layer "B.Cu") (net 19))
 (segment (start 184.09835 118.31135) (end 185.36835 117.04135) (width 0.762) (layer "B.Cu") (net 19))
 (segment (start 139.64835 120.85135) (end 139.64835 99.26135) (width 0.762) (layer "B.Cu") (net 19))
 (segment (start 114.88335 118.31135) (end 114.88335 124.66135) (width 0.762) (layer "B.Cu") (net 19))
 (segment (start 178.00335 121.48635) (end 178.00335 124.02635) (width 0.762) (layer "B.Cu") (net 19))
 (segment (start 125.04335 86.56135) (end 125.04335 91.64135) (width 0.762) (layer "B.Cu") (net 19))
 (segment (start 139.01335 87.19635) (end 138.37835 86.56135) (width 0.762) (layer "B.Cu") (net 19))
 (segment (start 116.15335 125.93135) (end 120.59835 125.93135) (width 0.762) (layer "B.Cu") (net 19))
 (segment (start 184.09835 122.75635) (end 180.92335 125.93135) (width 0.762) (layer "B.Cu") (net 19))
 (segment (start 114.88335 124.66135) (end 116.15335 125.93135) (width 0.762) (layer "B.Cu") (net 19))
 (segment (start 120.59835 125.93135) (end 124.40835 122.12135) (width 0.762) (layer "B.Cu") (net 19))
 (segment (start 124.40835 122.12135) (end 138.37835 122.12135) (width 0.762) (layer "B.Cu") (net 19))
 (segment (start 127.58335 119.58135) (end 130.75835 119.58135) (width 0.762) (layer "B.Cu") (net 15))
 (segment (start 127.58335 117.04135) (end 130.75835 117.04135) (width 0.762) (layer "B.Cu") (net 14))
 (segment (start 127.58335 114.50135) (end 130.75835 114.50135) (width 0.762) (layer "B.Cu") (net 13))
 (segment (start 127.58335 111.96135) (end 130.75835 111.96135) (width 0.762) (layer "B.Cu") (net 3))
 (segment (start 109.80335 89.10135) (end 112.34335 86.56135) (width 0.762) (layer "B.Cu") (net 21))
 (segment (start 111.96335 104.34135) (end 111.07335 104.34135) (width 0.762) (layer "B.Cu") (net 21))
 (segment (start 109.80335 103.07135) (end 109.80335 89.10135) (width 0.762) (layer "B.Cu") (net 21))
 (segment (start 112.34335 86.56135) (end 114.88335 86.56135) (width 0.762) (layer "B.Cu") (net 21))
 (segment (start 111.07335 104.34135) (end 109.80335 103.07135) (width 0.762) (layer "B.Cu") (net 21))
 (segment (start 163.14335 111.96135) (end 159.96835 108.78635) (width 0.762) (layer "B.Cu") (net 6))
 (segment (start 163.14335 117.67635) (end 163.14335 111.96135) (width 0.762) (layer "B.Cu") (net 6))
 (segment (start 160.60335 119.96135) (end 161.49335 120.85135) (width 0.762) (layer "B.Cu") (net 7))
 (segment (start 165.68335 117.67635) (end 165.68335 119.83635) (width 0.762) (layer "B.Cu") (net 7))
 (segment (start 165.68335 111.96135) (end 165.68335 117.67635) (width 0.762) (layer "B.Cu") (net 7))
 (segment (start 171.39835 111.32635) (end 166.31835 111.32635) (width 0.762) (layer "B.Cu") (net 7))
 (segment (start 166.31835 111.32635) (end 165.68335 111.96135) (width 0.762) (layer "B.Cu") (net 7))
 (segment (start 161.49335 120.85135) (end 164.66835 120.85135) (width 0.762) (layer "B.Cu") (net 7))
 (segment (start 164.66835 120.85135) (end 165.68335 119.83635) (width 0.762) (layer "B.Cu") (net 7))
 (segment (start 160.60335 117.67635) (end 160.60335 119.96135) (width 0.762) (layer "B.Cu") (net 7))
 (segment (start 173.93835 108.78635) (end 171.39835 111.32635) (width 0.762) (layer "B.Cu") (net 7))
 (segment (start 133.29835 91.64135) (end 134.56835 90.37135) (width 0.762) (layer "B.Cu") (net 18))
 (segment (start 134.56835 90.37135) (end 134.56835 89.10135) (width 0.762) (layer "B.Cu") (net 18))
 (segment (start 130.75835 91.64135) (end 133.29835 91.64135) (width 0.762) (layer "B.Cu") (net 18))
 (segment (start 137.10835 92.27635) (end 137.10835 89.10135) (width 0.762) (layer "B.Cu") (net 17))
 (segment (start 135.20335 94.18135) (end 137.10835 92.27635) (width 0.762) (layer "B.Cu") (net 17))
 (segment (start 130.75835 94.18135) (end 135.20335 94.18135) (width 0.762) (layer "B.Cu") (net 17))
 (via (at 172.92335 124.02635) (size 2.1844) (drill 1) (layers "F.Cu" "B.Cu") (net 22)))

